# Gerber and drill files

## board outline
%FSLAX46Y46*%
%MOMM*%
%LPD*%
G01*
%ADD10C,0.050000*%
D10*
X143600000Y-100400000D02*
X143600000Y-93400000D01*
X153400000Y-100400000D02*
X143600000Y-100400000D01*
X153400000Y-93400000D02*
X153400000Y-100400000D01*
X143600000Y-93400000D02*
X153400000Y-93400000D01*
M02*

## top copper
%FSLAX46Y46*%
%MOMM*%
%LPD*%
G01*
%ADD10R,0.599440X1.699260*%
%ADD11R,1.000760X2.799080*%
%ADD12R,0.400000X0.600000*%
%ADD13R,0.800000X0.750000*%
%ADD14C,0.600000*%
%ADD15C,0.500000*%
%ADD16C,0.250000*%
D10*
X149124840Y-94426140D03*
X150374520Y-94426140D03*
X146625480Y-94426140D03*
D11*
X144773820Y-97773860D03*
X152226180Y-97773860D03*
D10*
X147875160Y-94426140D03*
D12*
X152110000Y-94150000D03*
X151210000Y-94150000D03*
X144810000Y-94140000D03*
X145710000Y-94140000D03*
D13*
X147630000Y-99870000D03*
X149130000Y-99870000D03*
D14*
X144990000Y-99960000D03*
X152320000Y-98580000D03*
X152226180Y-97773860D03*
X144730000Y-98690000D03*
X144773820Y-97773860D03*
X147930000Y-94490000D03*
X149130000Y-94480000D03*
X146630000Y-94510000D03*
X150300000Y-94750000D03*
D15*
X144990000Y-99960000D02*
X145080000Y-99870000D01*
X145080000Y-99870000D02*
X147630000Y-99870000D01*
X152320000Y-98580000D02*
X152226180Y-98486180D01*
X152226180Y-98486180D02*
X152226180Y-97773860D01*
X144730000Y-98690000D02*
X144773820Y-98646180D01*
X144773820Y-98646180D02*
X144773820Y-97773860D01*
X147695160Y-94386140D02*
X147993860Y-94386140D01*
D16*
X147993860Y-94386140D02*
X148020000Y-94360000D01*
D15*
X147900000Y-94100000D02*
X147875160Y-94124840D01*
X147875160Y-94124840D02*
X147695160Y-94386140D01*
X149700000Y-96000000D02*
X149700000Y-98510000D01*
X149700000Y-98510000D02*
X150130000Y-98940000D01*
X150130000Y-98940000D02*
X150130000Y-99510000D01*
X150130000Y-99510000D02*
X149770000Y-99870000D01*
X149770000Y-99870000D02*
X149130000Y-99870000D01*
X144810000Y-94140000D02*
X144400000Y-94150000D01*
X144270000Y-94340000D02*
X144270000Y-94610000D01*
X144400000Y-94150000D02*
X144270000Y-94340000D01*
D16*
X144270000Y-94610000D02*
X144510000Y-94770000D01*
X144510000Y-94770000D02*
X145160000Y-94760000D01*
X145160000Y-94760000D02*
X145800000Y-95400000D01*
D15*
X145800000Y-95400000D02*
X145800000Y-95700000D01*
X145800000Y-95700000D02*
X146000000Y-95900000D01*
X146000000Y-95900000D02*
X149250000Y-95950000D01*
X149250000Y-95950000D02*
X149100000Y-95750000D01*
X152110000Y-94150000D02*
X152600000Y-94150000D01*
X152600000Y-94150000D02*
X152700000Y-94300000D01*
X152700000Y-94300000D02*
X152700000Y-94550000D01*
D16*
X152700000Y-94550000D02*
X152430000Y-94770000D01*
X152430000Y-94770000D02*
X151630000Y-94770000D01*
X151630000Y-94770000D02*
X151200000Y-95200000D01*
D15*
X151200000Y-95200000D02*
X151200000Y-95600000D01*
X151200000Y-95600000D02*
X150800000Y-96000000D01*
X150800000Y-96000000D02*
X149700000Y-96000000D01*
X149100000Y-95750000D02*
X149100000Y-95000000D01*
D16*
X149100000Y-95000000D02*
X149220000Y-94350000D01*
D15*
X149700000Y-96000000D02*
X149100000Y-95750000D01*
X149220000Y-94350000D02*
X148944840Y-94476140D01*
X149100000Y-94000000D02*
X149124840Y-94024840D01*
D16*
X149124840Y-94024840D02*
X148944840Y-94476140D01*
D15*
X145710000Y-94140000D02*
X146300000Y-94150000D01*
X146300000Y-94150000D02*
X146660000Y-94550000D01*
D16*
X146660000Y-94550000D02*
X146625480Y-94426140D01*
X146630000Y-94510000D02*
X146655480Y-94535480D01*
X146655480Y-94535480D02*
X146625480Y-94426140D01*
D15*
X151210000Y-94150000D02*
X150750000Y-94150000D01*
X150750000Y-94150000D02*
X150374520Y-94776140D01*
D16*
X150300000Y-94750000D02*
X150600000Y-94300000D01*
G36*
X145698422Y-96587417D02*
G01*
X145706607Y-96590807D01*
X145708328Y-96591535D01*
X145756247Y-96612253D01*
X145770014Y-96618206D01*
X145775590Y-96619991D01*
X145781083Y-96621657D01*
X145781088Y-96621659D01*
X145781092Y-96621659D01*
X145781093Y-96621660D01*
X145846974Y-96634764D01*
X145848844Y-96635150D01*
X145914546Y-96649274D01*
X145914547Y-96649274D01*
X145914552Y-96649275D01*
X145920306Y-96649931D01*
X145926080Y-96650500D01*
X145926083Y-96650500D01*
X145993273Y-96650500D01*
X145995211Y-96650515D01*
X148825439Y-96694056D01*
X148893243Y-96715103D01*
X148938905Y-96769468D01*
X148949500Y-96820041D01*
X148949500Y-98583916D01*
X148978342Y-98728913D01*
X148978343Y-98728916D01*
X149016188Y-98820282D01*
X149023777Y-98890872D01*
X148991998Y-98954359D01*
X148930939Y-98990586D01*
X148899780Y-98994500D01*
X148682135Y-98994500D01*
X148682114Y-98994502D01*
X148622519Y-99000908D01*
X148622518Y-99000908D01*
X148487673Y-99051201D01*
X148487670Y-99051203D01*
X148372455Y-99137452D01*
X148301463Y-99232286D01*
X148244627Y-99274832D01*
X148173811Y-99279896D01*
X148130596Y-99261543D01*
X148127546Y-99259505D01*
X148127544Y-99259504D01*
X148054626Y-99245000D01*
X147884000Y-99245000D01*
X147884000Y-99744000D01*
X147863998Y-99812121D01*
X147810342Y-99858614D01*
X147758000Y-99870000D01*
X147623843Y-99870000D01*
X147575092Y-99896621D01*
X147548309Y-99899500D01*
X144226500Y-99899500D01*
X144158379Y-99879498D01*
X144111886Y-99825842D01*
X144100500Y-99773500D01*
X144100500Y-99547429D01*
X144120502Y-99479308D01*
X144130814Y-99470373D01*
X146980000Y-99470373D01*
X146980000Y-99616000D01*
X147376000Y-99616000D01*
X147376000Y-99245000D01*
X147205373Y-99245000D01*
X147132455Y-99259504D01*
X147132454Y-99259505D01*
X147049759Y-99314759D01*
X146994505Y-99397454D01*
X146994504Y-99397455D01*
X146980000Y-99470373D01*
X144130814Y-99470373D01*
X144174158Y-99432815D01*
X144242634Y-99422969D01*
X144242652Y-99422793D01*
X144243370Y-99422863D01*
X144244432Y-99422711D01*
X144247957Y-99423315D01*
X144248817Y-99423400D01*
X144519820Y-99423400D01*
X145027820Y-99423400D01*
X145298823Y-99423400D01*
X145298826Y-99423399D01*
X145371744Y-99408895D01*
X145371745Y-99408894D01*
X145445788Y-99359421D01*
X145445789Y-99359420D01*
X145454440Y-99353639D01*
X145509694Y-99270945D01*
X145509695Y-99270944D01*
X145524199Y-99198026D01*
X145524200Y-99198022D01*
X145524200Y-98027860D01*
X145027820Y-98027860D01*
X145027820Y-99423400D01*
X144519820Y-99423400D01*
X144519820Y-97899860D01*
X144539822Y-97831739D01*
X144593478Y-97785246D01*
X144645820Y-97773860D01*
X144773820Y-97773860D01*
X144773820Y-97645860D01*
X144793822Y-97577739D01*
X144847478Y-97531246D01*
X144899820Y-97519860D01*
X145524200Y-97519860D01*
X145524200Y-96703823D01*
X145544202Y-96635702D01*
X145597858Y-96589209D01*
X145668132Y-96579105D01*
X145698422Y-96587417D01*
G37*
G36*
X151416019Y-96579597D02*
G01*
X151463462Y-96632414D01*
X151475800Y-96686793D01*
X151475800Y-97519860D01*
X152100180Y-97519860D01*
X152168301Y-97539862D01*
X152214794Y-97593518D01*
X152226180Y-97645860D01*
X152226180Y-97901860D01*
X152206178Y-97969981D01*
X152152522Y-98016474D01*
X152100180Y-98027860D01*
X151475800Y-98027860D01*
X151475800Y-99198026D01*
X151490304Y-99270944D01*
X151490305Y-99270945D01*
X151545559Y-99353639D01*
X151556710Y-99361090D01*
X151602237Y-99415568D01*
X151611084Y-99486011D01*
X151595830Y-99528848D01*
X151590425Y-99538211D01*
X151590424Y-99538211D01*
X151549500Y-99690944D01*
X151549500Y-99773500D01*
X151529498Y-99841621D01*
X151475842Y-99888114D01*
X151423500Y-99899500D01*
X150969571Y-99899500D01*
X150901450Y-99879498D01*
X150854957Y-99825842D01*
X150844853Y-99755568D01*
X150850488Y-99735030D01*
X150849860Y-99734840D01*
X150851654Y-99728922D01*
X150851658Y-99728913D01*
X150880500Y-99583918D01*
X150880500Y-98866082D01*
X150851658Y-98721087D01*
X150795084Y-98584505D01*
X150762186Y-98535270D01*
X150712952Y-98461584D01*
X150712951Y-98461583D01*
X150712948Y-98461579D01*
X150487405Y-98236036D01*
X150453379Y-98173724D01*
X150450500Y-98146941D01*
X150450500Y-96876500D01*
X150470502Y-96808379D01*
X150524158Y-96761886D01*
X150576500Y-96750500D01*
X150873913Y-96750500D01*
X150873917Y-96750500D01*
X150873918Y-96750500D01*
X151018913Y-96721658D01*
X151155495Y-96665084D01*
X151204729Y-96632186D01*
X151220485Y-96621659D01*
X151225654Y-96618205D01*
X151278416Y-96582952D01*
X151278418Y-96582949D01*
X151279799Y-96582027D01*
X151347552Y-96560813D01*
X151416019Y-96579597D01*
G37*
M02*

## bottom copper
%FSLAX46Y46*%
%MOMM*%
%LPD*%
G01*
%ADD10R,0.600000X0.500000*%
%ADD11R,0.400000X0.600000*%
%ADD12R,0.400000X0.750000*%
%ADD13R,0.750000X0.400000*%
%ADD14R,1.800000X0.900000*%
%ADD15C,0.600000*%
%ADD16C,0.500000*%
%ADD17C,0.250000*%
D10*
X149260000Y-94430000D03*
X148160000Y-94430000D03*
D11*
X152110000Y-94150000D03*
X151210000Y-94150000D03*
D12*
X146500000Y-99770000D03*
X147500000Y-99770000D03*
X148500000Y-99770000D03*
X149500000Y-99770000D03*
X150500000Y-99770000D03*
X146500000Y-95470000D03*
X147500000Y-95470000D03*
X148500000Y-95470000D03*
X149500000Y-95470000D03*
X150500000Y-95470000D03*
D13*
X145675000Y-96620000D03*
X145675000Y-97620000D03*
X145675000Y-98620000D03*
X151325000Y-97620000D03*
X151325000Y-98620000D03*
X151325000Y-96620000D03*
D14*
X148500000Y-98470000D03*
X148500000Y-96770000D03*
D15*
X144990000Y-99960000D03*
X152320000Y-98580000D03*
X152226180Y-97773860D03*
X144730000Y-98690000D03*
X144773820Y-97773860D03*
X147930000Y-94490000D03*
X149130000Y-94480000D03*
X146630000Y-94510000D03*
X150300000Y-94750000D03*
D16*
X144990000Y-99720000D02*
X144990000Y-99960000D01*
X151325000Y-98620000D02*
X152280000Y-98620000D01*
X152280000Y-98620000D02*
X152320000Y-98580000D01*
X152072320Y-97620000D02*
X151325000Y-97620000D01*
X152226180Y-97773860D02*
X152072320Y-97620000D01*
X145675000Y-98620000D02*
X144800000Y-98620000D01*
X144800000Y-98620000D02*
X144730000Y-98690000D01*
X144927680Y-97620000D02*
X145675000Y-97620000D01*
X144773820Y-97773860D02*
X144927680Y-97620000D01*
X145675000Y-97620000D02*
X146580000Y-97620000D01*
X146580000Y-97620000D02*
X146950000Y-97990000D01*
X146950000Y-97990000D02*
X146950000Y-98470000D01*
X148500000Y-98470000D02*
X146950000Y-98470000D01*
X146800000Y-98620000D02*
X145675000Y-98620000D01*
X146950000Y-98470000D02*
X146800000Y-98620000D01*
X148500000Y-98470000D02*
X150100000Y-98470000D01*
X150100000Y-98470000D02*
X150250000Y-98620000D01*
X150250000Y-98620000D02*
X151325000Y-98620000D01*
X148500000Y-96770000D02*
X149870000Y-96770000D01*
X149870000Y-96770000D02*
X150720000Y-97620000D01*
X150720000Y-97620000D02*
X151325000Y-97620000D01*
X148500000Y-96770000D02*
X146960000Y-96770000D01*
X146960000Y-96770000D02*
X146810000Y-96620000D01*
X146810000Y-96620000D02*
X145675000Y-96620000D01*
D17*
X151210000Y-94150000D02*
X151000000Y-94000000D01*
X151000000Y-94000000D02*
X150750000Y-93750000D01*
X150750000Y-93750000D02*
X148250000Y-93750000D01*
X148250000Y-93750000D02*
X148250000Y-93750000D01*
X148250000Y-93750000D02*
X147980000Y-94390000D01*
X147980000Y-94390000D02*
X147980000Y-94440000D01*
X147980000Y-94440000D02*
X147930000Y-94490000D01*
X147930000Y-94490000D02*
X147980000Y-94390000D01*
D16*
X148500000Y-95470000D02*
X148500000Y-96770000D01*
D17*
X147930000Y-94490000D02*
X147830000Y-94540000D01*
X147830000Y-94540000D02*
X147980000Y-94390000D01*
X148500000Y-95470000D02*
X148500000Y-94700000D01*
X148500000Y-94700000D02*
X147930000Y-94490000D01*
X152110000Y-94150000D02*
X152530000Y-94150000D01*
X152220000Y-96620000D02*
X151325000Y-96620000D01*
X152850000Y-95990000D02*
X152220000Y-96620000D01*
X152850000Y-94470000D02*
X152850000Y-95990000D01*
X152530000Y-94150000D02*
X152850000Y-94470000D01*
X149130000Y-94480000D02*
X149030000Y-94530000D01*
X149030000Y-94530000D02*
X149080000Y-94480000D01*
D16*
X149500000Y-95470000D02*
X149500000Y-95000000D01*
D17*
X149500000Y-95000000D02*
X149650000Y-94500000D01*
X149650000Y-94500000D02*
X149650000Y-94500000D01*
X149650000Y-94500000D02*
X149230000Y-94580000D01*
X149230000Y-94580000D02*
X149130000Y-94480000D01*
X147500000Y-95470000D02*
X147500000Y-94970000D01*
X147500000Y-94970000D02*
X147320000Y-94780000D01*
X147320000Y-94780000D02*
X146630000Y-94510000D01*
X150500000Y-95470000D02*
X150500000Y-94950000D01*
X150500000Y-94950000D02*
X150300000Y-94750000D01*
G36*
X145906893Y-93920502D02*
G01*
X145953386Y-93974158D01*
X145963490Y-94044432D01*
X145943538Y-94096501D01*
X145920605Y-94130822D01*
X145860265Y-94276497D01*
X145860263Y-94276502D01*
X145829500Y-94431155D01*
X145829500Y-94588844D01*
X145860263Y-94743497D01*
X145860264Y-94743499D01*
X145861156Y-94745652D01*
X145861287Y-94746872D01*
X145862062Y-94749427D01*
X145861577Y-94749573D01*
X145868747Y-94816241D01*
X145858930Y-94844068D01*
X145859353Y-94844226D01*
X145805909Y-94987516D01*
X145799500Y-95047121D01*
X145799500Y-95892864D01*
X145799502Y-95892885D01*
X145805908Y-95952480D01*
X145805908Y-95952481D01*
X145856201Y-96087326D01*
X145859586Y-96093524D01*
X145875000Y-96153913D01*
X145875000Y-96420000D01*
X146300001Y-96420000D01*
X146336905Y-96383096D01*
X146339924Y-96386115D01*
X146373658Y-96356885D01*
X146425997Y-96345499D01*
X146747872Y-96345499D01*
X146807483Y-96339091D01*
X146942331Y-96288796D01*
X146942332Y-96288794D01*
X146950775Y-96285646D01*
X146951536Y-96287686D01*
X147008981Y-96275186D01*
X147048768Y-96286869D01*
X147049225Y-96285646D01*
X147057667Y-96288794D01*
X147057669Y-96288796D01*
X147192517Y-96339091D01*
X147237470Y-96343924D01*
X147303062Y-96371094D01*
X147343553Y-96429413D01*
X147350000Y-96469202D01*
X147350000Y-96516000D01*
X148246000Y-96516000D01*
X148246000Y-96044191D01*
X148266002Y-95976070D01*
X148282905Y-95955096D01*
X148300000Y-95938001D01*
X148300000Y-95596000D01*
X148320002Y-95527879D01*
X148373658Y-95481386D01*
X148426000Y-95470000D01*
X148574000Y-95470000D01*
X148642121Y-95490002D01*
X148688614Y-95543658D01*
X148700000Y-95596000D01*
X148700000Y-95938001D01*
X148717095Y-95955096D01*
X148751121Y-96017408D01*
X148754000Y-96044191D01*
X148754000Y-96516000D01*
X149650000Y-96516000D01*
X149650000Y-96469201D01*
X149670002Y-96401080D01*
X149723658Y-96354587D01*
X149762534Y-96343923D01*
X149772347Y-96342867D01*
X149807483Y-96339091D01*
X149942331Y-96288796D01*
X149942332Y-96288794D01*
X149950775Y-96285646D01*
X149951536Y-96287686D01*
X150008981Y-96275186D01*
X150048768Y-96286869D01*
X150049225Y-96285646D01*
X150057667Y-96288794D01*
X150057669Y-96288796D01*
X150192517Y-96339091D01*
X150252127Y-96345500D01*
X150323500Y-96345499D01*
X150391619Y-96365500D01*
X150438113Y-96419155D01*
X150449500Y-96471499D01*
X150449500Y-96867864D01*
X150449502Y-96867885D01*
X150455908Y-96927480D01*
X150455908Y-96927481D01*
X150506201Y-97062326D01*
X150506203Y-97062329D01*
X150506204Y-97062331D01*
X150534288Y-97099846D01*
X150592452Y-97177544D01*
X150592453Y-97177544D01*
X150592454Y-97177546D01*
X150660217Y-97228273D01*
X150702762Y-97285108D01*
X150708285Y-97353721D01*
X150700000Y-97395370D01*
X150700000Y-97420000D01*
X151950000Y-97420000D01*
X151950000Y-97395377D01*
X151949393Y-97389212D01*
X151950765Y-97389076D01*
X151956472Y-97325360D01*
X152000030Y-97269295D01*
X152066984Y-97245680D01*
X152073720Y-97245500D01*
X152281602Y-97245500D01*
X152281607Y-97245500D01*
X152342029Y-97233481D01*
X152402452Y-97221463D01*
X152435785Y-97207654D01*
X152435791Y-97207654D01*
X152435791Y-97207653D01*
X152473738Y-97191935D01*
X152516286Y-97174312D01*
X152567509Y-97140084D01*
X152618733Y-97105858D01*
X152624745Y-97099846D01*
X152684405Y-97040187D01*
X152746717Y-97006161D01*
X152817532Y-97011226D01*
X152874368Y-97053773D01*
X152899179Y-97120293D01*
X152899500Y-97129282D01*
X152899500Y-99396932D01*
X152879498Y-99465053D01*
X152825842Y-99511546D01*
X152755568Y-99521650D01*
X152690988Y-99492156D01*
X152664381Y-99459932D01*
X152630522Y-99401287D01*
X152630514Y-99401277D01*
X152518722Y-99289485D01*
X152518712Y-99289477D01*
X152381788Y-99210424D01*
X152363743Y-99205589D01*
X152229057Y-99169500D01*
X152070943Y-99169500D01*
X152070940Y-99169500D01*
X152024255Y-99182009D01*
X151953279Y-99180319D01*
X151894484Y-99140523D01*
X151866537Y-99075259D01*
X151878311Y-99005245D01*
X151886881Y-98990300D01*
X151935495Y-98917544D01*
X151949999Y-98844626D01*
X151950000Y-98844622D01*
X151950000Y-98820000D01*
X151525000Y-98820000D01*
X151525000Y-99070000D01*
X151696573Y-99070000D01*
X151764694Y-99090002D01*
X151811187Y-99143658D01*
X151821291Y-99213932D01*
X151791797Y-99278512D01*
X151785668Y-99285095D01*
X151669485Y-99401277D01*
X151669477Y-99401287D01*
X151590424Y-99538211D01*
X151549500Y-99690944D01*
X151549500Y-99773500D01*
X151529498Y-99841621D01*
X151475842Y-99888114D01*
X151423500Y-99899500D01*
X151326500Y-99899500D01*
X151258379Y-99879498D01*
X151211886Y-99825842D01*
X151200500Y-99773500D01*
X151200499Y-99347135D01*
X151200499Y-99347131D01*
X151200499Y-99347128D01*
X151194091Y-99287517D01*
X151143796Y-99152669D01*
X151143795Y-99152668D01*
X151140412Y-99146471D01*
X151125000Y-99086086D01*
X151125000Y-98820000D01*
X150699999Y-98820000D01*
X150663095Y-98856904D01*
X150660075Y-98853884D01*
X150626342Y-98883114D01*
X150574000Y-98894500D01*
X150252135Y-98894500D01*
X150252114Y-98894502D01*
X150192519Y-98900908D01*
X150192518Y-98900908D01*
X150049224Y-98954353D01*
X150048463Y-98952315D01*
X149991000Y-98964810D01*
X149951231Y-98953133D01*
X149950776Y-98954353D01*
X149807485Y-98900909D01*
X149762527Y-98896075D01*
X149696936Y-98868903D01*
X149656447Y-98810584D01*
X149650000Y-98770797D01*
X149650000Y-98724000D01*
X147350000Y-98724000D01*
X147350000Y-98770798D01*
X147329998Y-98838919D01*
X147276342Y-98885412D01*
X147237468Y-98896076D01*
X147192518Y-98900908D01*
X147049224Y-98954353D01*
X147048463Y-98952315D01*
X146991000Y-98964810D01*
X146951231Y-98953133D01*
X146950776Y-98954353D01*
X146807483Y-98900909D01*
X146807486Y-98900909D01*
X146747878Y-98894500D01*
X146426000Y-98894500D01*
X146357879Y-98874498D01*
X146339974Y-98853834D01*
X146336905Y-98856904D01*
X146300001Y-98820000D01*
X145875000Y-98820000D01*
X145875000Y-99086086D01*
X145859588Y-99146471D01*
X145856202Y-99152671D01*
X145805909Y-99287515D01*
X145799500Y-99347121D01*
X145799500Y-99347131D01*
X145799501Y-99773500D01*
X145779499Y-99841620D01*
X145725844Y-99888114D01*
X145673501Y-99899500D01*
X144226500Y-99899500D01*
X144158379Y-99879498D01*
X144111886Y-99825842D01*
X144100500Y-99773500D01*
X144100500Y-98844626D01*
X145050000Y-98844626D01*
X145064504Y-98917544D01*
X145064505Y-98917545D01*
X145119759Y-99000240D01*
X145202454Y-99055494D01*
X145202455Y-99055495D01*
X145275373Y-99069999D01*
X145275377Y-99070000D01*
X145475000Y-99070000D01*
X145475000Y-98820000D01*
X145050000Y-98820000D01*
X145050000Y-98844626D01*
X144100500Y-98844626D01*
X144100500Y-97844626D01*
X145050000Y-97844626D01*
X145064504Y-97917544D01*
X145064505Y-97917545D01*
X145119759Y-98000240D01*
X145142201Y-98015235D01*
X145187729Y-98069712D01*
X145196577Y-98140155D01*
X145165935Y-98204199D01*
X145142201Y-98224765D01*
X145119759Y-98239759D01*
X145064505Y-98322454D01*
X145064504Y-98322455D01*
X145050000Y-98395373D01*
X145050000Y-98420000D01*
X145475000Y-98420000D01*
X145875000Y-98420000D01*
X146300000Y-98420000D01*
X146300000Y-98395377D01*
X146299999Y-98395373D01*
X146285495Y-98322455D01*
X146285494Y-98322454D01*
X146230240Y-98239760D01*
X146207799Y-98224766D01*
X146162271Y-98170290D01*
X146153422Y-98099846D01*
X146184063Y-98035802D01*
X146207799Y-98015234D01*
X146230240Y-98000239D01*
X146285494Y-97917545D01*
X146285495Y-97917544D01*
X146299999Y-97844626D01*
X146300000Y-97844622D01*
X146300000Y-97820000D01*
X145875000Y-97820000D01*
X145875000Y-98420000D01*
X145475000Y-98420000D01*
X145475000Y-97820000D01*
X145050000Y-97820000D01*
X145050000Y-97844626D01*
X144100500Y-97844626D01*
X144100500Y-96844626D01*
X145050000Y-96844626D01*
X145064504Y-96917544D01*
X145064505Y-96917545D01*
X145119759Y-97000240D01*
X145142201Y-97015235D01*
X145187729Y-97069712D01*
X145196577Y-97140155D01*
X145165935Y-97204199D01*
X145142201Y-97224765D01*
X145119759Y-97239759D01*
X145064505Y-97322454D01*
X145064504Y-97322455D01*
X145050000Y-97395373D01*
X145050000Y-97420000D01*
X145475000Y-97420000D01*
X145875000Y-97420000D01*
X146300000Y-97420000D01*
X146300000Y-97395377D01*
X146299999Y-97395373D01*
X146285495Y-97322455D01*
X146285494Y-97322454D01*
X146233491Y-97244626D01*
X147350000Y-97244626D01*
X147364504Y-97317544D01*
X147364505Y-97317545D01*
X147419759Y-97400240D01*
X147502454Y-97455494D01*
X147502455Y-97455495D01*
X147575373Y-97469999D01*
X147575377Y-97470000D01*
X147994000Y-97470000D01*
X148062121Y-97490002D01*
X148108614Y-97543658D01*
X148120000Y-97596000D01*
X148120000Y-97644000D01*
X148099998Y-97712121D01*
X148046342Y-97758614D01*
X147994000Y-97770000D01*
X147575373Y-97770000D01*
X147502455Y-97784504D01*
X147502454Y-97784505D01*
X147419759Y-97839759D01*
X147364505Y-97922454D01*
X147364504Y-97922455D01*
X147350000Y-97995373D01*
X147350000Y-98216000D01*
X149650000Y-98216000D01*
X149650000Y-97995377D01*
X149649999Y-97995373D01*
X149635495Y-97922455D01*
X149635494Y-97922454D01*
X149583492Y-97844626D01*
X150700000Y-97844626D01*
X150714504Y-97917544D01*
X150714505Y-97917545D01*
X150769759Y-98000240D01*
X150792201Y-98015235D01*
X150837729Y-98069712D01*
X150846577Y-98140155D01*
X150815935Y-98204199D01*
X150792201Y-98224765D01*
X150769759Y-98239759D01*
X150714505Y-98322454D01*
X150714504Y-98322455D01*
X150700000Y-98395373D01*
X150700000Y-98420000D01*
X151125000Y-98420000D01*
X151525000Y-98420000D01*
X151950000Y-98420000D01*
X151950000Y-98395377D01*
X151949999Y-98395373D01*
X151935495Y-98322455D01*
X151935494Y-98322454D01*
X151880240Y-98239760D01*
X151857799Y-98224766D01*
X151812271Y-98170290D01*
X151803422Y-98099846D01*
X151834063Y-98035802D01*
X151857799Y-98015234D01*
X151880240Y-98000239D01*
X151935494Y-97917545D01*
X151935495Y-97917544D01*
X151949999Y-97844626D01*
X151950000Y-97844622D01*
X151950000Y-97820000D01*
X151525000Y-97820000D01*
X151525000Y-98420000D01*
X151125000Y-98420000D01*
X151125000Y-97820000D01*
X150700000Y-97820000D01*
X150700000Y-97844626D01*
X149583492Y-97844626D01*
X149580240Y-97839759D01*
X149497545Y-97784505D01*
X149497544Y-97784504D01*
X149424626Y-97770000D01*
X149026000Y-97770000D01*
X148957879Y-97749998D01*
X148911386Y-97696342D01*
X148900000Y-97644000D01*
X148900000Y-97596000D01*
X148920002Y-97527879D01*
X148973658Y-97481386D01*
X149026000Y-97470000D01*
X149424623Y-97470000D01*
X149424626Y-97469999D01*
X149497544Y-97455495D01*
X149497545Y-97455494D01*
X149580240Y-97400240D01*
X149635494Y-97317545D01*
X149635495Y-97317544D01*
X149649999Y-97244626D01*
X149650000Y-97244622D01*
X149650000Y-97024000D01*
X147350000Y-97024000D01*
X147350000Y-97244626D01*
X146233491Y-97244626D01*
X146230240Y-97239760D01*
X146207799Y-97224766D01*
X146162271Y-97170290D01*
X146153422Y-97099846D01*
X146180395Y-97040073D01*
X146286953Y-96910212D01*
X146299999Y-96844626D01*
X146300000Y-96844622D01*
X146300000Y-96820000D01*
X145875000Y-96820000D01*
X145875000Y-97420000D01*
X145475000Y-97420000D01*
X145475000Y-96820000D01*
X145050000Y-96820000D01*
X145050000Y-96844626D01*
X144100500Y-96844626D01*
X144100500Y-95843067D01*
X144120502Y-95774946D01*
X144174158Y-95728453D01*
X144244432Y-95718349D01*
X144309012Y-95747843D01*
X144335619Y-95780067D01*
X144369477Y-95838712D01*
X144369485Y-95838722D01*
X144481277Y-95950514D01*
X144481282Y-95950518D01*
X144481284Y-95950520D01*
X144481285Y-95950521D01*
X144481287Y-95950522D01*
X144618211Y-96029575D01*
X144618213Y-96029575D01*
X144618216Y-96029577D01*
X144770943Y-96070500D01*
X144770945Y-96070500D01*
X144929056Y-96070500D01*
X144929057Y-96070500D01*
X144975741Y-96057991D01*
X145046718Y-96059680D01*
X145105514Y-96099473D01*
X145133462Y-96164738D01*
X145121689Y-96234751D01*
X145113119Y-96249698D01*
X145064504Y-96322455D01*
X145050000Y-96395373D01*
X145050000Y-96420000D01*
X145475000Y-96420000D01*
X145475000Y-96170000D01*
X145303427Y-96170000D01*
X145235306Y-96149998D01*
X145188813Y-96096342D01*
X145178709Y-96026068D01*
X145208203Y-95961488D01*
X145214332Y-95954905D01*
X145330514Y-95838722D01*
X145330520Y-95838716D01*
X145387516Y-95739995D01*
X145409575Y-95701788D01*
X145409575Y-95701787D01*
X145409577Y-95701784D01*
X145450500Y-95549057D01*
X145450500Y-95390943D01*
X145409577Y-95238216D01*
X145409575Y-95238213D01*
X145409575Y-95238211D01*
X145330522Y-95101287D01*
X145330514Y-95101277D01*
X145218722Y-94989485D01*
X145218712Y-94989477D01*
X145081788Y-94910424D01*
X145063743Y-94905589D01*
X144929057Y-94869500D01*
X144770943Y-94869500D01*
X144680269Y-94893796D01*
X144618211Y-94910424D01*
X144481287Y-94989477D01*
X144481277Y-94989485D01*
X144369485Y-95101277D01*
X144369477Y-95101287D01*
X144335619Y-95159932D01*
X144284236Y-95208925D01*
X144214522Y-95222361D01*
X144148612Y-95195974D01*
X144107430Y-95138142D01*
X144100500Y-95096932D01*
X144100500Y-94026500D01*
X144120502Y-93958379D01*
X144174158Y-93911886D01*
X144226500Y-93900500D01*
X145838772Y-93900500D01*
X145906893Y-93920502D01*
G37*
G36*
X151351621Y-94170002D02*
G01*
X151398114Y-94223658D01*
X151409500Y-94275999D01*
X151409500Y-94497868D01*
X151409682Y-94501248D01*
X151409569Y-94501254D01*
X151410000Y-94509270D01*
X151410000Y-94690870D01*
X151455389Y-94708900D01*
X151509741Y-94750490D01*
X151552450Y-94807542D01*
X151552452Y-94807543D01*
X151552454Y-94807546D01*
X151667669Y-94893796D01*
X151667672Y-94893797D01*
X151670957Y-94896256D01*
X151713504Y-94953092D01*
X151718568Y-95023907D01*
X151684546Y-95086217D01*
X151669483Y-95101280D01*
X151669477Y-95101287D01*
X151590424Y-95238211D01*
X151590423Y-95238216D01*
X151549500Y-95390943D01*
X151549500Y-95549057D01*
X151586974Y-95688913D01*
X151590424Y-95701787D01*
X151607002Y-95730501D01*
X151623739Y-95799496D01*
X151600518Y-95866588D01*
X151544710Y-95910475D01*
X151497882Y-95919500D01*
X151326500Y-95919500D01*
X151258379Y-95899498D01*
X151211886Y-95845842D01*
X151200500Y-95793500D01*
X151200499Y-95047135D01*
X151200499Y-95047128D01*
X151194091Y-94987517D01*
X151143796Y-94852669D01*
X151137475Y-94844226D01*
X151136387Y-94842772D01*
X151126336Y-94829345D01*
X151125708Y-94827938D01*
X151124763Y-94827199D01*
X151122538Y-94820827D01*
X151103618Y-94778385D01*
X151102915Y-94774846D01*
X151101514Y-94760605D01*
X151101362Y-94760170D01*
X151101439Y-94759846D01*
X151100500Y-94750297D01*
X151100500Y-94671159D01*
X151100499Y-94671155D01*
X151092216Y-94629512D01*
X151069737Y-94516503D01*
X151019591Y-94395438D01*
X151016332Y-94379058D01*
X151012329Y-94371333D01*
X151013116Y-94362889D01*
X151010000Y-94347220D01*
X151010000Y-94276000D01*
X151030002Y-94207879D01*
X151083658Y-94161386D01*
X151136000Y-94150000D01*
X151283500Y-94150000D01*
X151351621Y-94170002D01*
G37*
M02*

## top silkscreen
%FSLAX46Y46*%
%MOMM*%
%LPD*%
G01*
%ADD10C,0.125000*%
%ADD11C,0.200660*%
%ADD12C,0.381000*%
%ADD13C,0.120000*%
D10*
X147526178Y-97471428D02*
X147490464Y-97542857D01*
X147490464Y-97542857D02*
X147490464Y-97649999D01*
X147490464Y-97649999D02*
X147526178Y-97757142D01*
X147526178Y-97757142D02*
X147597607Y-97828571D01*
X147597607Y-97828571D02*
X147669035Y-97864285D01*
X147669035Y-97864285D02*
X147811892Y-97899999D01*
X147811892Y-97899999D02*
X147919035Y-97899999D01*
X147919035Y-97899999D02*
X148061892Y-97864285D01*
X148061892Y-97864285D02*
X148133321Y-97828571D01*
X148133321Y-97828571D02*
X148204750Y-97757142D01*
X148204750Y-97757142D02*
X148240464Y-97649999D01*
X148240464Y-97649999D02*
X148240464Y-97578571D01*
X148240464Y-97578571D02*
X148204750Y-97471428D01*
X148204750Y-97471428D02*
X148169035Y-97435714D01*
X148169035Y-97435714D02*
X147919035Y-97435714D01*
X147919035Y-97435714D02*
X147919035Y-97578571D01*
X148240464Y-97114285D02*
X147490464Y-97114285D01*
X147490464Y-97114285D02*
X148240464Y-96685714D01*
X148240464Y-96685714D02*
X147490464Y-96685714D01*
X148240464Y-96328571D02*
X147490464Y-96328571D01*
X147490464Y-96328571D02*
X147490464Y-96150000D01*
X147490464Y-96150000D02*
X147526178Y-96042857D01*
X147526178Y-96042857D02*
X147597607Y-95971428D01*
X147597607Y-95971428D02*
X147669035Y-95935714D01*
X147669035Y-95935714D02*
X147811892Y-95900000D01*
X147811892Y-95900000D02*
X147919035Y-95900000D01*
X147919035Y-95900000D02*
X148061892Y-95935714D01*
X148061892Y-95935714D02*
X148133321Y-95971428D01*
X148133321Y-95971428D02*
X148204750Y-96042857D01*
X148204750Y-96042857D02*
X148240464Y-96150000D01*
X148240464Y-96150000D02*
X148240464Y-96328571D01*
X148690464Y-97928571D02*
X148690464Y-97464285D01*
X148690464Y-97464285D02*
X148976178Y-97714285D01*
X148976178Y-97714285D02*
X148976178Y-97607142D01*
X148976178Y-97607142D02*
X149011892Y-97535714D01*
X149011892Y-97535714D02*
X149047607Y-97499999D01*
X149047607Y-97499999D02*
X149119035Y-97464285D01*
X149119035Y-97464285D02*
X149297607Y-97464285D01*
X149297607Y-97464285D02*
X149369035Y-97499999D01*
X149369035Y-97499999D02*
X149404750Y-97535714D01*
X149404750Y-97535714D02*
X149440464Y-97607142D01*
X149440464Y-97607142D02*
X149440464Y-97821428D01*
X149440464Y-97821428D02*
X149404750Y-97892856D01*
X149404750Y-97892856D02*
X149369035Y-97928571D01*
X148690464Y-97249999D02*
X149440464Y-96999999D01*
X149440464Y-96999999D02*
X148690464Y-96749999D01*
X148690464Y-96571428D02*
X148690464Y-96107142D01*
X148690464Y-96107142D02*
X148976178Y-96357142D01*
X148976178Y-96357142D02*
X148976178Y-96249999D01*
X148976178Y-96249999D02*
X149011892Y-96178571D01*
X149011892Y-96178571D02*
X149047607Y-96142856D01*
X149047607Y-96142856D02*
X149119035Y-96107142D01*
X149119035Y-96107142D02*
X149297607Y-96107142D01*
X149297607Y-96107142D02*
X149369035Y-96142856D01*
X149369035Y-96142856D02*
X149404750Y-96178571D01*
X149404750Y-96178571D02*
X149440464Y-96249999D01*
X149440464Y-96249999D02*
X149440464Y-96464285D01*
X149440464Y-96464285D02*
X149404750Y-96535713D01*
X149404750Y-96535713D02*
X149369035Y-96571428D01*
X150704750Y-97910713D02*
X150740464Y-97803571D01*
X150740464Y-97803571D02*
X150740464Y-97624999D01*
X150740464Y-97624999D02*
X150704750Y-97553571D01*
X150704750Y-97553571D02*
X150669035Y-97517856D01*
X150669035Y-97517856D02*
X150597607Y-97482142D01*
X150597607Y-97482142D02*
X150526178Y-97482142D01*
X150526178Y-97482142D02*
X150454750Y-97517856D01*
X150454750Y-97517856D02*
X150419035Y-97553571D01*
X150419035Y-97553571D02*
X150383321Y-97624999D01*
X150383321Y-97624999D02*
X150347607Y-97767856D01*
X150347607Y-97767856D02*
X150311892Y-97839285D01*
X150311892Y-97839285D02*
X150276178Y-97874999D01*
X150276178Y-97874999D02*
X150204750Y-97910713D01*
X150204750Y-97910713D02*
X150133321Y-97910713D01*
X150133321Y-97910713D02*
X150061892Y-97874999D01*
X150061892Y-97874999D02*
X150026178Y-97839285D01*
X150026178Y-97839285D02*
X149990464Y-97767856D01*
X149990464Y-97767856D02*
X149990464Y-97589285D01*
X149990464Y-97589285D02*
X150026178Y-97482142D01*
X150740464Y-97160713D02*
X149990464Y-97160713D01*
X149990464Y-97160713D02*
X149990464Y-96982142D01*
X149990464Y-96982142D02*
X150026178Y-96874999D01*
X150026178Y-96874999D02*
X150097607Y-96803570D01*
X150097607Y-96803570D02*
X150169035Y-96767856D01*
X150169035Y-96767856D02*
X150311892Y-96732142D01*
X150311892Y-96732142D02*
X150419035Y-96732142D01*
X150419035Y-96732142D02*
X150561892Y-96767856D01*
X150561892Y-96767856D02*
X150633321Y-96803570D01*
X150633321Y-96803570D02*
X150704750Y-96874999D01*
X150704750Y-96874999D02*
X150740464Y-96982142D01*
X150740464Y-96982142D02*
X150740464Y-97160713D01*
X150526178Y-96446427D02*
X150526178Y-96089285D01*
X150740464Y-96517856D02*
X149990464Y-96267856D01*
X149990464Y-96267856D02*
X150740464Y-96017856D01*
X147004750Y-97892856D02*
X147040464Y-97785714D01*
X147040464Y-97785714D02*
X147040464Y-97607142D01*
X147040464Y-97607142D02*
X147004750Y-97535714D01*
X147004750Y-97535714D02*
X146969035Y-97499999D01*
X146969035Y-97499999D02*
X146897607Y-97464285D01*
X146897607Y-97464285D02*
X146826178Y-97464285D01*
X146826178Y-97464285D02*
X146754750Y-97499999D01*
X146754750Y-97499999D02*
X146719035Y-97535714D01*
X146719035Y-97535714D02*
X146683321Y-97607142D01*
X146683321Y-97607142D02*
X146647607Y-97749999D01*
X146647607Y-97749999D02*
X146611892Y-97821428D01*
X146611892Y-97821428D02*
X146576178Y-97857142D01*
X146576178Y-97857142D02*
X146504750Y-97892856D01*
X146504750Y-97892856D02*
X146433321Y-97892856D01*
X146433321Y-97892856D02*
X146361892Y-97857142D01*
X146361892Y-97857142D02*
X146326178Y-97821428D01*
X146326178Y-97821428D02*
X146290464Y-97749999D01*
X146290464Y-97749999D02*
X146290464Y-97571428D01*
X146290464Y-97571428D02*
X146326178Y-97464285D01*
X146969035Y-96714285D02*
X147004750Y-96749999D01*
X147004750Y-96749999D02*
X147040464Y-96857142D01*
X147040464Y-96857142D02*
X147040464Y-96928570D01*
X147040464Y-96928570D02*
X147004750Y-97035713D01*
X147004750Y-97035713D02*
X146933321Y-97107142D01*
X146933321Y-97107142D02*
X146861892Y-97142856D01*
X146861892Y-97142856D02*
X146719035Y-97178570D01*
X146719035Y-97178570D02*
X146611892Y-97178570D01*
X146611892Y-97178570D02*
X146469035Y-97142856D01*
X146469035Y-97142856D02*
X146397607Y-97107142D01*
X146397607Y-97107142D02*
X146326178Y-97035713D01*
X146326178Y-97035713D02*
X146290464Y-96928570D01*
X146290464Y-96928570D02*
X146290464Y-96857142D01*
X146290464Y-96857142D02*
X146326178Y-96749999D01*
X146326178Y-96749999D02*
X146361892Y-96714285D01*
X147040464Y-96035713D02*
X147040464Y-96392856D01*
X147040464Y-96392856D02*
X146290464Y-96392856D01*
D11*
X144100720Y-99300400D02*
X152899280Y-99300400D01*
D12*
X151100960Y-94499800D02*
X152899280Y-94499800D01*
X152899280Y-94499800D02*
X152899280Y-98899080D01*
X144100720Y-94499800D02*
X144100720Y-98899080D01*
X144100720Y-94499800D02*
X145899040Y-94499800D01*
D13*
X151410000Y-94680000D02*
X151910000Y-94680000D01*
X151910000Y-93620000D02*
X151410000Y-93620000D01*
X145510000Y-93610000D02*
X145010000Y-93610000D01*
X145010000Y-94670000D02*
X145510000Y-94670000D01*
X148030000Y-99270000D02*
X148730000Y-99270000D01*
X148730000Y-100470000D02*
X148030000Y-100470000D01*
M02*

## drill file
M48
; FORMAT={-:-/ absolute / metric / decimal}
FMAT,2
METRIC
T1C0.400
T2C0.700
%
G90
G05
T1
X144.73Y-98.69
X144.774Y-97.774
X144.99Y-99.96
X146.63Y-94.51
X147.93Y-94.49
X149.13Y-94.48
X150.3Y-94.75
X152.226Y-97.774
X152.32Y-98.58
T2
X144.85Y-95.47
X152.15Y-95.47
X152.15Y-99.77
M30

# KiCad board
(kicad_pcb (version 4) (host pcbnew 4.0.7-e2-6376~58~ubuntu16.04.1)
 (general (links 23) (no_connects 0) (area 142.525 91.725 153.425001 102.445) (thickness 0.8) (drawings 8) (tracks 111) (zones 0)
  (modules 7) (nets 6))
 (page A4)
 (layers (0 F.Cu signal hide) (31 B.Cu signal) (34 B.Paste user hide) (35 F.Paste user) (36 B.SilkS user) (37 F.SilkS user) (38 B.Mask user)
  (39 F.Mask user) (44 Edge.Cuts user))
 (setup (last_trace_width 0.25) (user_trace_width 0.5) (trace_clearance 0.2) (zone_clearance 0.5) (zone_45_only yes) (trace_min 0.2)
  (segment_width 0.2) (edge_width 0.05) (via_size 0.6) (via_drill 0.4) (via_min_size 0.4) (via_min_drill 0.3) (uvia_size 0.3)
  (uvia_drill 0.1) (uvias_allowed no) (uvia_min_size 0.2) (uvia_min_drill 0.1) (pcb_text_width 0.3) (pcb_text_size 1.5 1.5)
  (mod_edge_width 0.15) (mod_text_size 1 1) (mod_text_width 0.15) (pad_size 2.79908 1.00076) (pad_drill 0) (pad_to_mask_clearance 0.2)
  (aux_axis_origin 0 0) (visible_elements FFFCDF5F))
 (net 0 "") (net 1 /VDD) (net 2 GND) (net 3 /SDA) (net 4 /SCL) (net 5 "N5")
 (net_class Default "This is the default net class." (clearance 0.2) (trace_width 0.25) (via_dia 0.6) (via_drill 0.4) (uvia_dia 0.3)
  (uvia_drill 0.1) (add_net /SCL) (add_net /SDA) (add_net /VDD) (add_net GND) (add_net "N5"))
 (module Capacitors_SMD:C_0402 (layer B.Cu) (at 148.71 94.43 180)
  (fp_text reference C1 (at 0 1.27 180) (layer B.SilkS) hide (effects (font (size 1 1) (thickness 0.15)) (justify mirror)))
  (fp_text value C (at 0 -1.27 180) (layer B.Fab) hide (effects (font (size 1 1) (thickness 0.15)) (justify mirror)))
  (pad 1 smd rect (at -0.55 0 180) (size 0.6 0.5) (layers B.Cu B.Paste B.Mask) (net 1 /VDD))
  (pad 2 smd rect (at 0.55 0 180) (size 0.6 0.5) (layers B.Cu B.Paste B.Mask) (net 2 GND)))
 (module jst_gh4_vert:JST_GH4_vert (layer F.Cu) (at 148.5 96.1 90)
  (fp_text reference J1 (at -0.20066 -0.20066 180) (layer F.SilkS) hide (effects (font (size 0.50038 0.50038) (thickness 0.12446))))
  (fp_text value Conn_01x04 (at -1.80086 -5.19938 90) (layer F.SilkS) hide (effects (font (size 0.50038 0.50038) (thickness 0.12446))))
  (fp_line (start -3.2004 -4.39928) (end -3.2004 4.39928) (layer F.SilkS) (width 0.20066))
  (fp_line (start 1.6002 2.60096) (end 1.6002 4.39928) (layer F.SilkS) (width 0.381))
  (fp_line (start 1.6002 4.39928) (end -2.79908 4.39928) (layer F.SilkS) (width 0.381))
  (fp_line (start 1.6002 -4.39928) (end -2.79908 -4.39928) (layer F.SilkS) (width 0.381))
  (fp_line (start 1.6002 -4.39928) (end 1.6002 -2.60096) (layer F.SilkS) (width 0.381))
  (pad 3 smd rect (at 1.67386 0.62484) (size 0.59944 1.69926) (layers F.Cu F.Paste F.Mask) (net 1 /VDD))
  (pad 4 smd rect (at 1.67386 1.87452) (size 0.59944 1.69926) (layers F.Cu F.Paste F.Mask) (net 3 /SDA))
  (pad 1 smd rect (at 1.67386 -1.87452) (size 0.59944 1.69926) (layers F.Cu F.Paste F.Mask) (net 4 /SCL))
  (pad "" smd rect (at -1.67386 -3.72618 90) (size 2.79908 1.00076) (layers F.Cu F.Paste F.Mask) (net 2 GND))
  (pad "" smd rect (at -1.67386 3.72618 90) (size 2.79908 1.00076) (layers F.Cu F.Paste F.Mask) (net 2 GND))
  (pad 2 smd rect (at 1.67386 -0.62484) (size 0.59944 1.69926) (layers F.Cu F.Paste F.Mask) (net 2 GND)))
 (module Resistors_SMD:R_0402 (layer F.Cu) (at 151.66 94.15 180)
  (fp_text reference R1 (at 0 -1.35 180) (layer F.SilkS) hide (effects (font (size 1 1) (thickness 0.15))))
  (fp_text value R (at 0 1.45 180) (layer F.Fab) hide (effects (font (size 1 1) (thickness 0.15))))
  (fp_line (start 0.25 -0.53) (end -0.25 -0.53) (layer F.SilkS) (width 0.12))
  (fp_line (start -0.25 0.53) (end 0.25 0.53) (layer F.SilkS) (width 0.12))
  (pad 1 smd rect (at -0.45 0 180) (size 0.4 0.6) (layers F.Cu F.Paste F.Mask) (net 1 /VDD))
  (pad 2 smd rect (at 0.45 0 180) (size 0.4 0.6) (layers F.Cu F.Paste F.Mask) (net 3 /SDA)))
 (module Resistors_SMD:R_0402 (layer F.Cu) (at 145.26 94.14)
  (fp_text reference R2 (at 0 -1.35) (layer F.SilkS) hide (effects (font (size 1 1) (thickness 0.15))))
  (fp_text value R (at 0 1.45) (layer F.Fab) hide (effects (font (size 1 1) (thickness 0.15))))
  (fp_line (start 0.25 -0.53) (end -0.25 -0.53) (layer F.SilkS) (width 0.12))
  (fp_line (start -0.25 0.53) (end 0.25 0.53) (layer F.SilkS) (width 0.12))
  (pad 1 smd rect (at -0.45 0) (size 0.4 0.6) (layers F.Cu F.Paste F.Mask) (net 1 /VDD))
  (pad 2 smd rect (at 0.45 0) (size 0.4 0.6) (layers F.Cu F.Paste F.Mask) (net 4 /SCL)))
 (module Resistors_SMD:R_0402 (layer B.Cu) (at 151.66 94.15 180)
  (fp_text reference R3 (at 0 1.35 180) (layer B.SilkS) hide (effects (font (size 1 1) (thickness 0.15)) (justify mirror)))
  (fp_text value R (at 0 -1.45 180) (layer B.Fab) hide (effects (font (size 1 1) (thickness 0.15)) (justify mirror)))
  (pad 1 smd rect (at -0.45 0 180) (size 0.4 0.6) (layers B.Cu B.Paste B.Mask) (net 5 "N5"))
  (pad 2 smd rect (at 0.45 0 180) (size 0.4 0.6) (layers B.Cu B.Paste B.Mask) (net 2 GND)))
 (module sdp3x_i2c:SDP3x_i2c (layer B.Cu) (at 148.5 97.62)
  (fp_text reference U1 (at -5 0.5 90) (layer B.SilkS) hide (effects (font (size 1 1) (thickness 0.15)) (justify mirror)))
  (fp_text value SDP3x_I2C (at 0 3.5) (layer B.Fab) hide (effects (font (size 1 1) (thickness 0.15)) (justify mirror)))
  (pad 16 smd rect (at -2 2.15) (size 0.4 0.75) (layers B.Cu B.Paste B.Mask))
  (pad 15 smd rect (at -1 2.15) (size 0.4 0.75) (layers B.Cu B.Paste B.Mask))
  (pad 14 smd rect (at 0 2.15) (size 0.4 0.75) (layers B.Cu B.Paste B.Mask))
  (pad 13 smd rect (at 1 2.15) (size 0.4 0.75) (layers B.Cu B.Paste B.Mask))
  (pad 12 smd rect (at 2 2.15) (size 0.4 0.75) (layers B.Cu B.Paste B.Mask))
  (pad 4 smd rect (at -2 -2.15) (size 0.4 0.75) (layers B.Cu B.Paste B.Mask))
  (pad 5 smd rect (at -1 -2.15) (size 0.4 0.75) (layers B.Cu B.Paste B.Mask) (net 4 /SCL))
  (pad 6 smd rect (at 0 -2.15) (size 0.4 0.75) (layers B.Cu B.Paste B.Mask) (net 2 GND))
  (pad 7 smd rect (at 1 -2.15) (size 0.4 0.75) (layers B.Cu B.Paste B.Mask) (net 1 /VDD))
  (pad 8 smd rect (at 2 -2.15) (size 0.4 0.75) (layers B.Cu B.Paste B.Mask) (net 3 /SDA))
  (pad 3 smd rect (at -2.825 -1) (size 0.75 0.4) (layers B.Cu B.Paste B.Mask) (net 2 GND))
  (pad 2 smd rect (at -2.825 0) (size 0.75 0.4) (layers B.Cu B.Paste B.Mask) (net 2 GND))
  (pad 1 smd rect (at -2.825 1) (size 0.75 0.4) (layers B.Cu B.Paste B.Mask) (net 2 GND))
  (pad 10 smd rect (at 2.825 0) (size 0.75 0.4) (layers B.Cu B.Paste B.Mask) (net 2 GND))
  (pad 11 smd rect (at 2.825 1) (size 0.75 0.4) (layers B.Cu B.Paste B.Mask) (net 2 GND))
  (pad 9 smd rect (at 2.825 -1) (size 0.75 0.4) (layers B.Cu B.Paste B.Mask) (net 5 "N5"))
  (pad 1 smd rect (at 0 0.85) (size 1.8 0.9) (layers B.Cu B.Paste B.Mask) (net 2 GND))
  (pad 1 smd rect (at 0 -0.85) (size 1.8 0.9) (layers B.Cu B.Paste B.Mask) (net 2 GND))
  (pad "" np_thru_hole circle (at 3.65 -2.15) (size 0.7 0.7) (drill 0.7) (layers *.Cu *.Mask) (zone_connect 0))
  (pad "" np_thru_hole circle (at 3.65 2.15) (size 0.7 0.7) (drill 0.7) (layers *.Cu *.Mask))
  (pad "" np_thru_hole circle (at -3.65 -2.15) (size 0.7 0.7) (drill 0.7) (layers *.Cu *.Mask)))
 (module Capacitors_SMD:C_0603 (layer F.Cu) (at 148.38 99.87 180)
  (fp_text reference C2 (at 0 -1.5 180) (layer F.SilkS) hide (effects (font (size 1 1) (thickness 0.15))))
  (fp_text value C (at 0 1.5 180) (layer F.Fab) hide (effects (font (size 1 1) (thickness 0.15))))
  (fp_line (start 0.35 0.6) (end -0.35 0.6) (layer F.SilkS) (width 0.12))
  (fp_line (start -0.35 -0.6) (end 0.35 -0.6) (layer F.SilkS) (width 0.12))
  (pad 2 smd rect (at 0.75 0 180) (size 0.8 0.75) (layers F.Cu F.Paste F.Mask) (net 2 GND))
  (pad 1 smd rect (at -0.75 0 180) (size 0.8 0.75) (layers F.Cu F.Paste F.Mask) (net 1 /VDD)))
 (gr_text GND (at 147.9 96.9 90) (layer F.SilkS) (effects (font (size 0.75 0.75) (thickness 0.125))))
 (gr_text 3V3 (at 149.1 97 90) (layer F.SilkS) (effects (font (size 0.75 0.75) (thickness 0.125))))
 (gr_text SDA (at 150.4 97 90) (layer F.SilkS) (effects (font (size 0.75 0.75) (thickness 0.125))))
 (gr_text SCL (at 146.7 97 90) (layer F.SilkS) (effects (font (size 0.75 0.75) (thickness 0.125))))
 (gr_line (start 143.6 100.4) (end 143.6 93.4) (angle 90) (layer Edge.Cuts) (width 0.05))
 (gr_line (start 153.4 100.4) (end 143.6 100.4) (angle 90) (layer Edge.Cuts) (width 0.05))
 (gr_line (start 153.4 93.4) (end 153.4 100.4) (angle 90) (layer Edge.Cuts) (width 0.05))
 (gr_line (start 143.6 93.4) (end 153.4 93.4) (angle 90) (layer Edge.Cuts) (width 0.05))
 (segment (start 144.99 99.72) (end 144.99 99.96) (width 0.5) (layer B.Cu) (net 2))
 (via (at 144.99 99.96) (size 0.6) (drill 0.4) (layers F.Cu B.Cu) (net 2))
 (segment (start 144.99 99.96) (end 145.08 99.87) (width 0.5) (layer F.Cu) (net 2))
 (segment (start 145.08 99.87) (end 147.63 99.87) (width 0.5) (layer F.Cu) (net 2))
 (segment (start 151.325 98.62) (end 152.28 98.62) (width 0.5) (layer B.Cu) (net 2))
 (segment (start 152.28 98.62) (end 152.32 98.58) (width 0.5) (layer B.Cu) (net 2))
 (via (at 152.32 98.58) (size 0.6) (drill 0.4) (layers F.Cu B.Cu) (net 2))
 (segment (start 152.32 98.58) (end 152.22618 98.48618) (width 0.5) (layer F.Cu) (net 2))
 (segment (start 152.22618 98.48618) (end 152.22618 97.77386) (width 0.5) (layer F.Cu) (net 2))
 (segment (start 152.07232 97.62) (end 151.325 97.62) (width 0.5) (layer B.Cu) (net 2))
 (segment (start 152.22618 97.77386) (end 152.07232 97.62) (width 0.5) (layer B.Cu) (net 2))
 (via (at 152.22618 97.77386) (size 0.6) (drill 0.4) (layers F.Cu B.Cu) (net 2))
 (segment (start 145.675 98.62) (end 144.8 98.62) (width 0.5) (layer B.Cu) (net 2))
 (segment (start 144.8 98.62) (end 144.73 98.69) (width 0.5) (layer B.Cu) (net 2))
 (via (at 144.73 98.69) (size 0.6) (drill 0.4) (layers F.Cu B.Cu) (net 2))
 (segment (start 144.73 98.69) (end 144.77382 98.64618) (width 0.5) (layer F.Cu) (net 2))
 (segment (start 144.77382 98.64618) (end 144.77382 97.77386) (width 0.5) (layer F.Cu) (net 2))
 (segment (start 144.92768 97.62) (end 145.675 97.62) (width 0.5) (layer B.Cu) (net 2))
 (segment (start 144.77382 97.77386) (end 144.92768 97.62) (width 0.5) (layer B.Cu) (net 2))
 (via (at 144.77382 97.77386) (size 0.6) (drill 0.4) (layers F.Cu B.Cu) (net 2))
 (segment (start 145.675 97.62) (end 146.58 97.62) (width 0.5) (layer B.Cu) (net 2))
 (segment (start 146.58 97.62) (end 146.95 97.99) (width 0.5) (layer B.Cu) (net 2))
 (segment (start 146.95 97.99) (end 146.95 98.47) (width 0.5) (layer B.Cu) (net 2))
 (segment (start 148.5 98.47) (end 146.95 98.47) (width 0.5) (layer B.Cu) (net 2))
 (segment (start 146.8 98.62) (end 145.675 98.62) (width 0.5) (layer B.Cu) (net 2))
 (segment (start 146.95 98.47) (end 146.8 98.62) (width 0.5) (layer B.Cu) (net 2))
 (segment (start 148.5 98.47) (end 150.1 98.47) (width 0.5) (layer B.Cu) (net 2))
 (segment (start 150.1 98.47) (end 150.25 98.62) (width 0.5) (layer B.Cu) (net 2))
 (segment (start 150.25 98.62) (end 151.325 98.62) (width 0.5) (layer B.Cu) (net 2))
 (segment (start 148.5 96.77) (end 149.87 96.77) (width 0.5) (layer B.Cu) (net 2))
 (segment (start 149.87 96.77) (end 150.72 97.62) (width 0.5) (layer B.Cu) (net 2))
 (segment (start 150.72 97.62) (end 151.325 97.62) (width 0.5) (layer B.Cu) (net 2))
 (segment (start 148.5 96.77) (end 146.96 96.77) (width 0.5) (layer B.Cu) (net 2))
 (segment (start 146.96 96.77) (end 146.81 96.62) (width 0.5) (layer B.Cu) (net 2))
 (segment (start 146.81 96.62) (end 145.675 96.62) (width 0.5) (layer B.Cu) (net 2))
 (segment (start 151.21 94.15) (end 151 94) (width 0.25) (layer B.Cu) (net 2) (status 10))
 (segment (start 151 94) (end 150.75 93.75) (width 0.25) (layer B.Cu) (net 2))
 (segment (start 150.75 93.75) (end 148.25 93.75) (width 0.25) (layer B.Cu) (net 2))
 (segment (start 148.25 93.75) (end 148.25 93.75) (width 0.25) (layer B.Cu) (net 2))
 (segment (start 148.25 93.75) (end 147.98 94.39) (width 0.25) (layer B.Cu) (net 2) (status 20))
 (segment (start 147.69516 94.38614) (end 147.99386 94.38614) (width 0.5) (layer F.Cu) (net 2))
 (segment (start 147.99386 94.38614) (end 148.02 94.36) (width 0.25) (layer F.Cu) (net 2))
 (via (at 147.93 94.49) (size 0.6) (drill 0.4) (layers F.Cu B.Cu) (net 2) (status 30))
 (segment (start 147.98 94.39) (end 147.98 94.44) (width 0.25) (layer B.Cu) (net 2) (status 30))
 (segment (start 147.98 94.44) (end 147.93 94.49) (width 0.25) (layer B.Cu) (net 2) (status 30))
 (segment (start 147.93 94.49) (end 147.98 94.39) (width 0.25) (layer B.Cu) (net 2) (status 30))
 (segment (start 148.5 95.47) (end 148.5 96.77) (width 0.5) (layer B.Cu) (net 2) (status 30))
 (segment (start 147.9 94.1) (end 147.87516 94.12484) (width 0.5) (layer F.Cu) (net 2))
 (segment (start 147.87516 94.12484) (end 147.69516 94.38614) (width 0.5) (layer F.Cu) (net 2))
 (segment (start 147.93 94.49) (end 147.83 94.54) (width 0.25) (layer B.Cu) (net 2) (status 30))
 (segment (start 147.83 94.54) (end 147.98 94.39) (width 0.25) (layer B.Cu) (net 2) (status 30))
 (segment (start 148.5 95.47) (end 148.5 94.7) (width 0.25) (layer B.Cu) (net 2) (status 10))
 (segment (start 148.5 94.7) (end 147.93 94.49) (width 0.25) (layer B.Cu) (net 2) (status 20))
 (segment (start 152.11 94.15) (end 152.53 94.15) (width 0.25) (layer B.Cu) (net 5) (status 10))
 (segment (start 152.22 96.62) (end 151.325 96.62) (width 0.25) (layer B.Cu) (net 5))
 (segment (start 152.85 95.99) (end 152.22 96.62) (width 0.25) (layer B.Cu) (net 5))
 (segment (start 152.85 94.47) (end 152.85 95.99) (width 0.25) (layer B.Cu) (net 5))
 (segment (start 152.53 94.15) (end 152.85 94.47) (width 0.25) (layer B.Cu) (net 5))
 (segment (start 149.7 96) (end 149.7 98.51) (width 0.5) (layer F.Cu) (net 1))
 (segment (start 149.7 98.51) (end 150.13 98.94) (width 0.5) (layer F.Cu) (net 1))
 (segment (start 150.13 98.94) (end 150.13 99.51) (width 0.5) (layer F.Cu) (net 1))
 (segment (start 150.13 99.51) (end 149.77 99.87) (width 0.5) (layer F.Cu) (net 1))
 (segment (start 149.77 99.87) (end 149.13 99.87) (width 0.5) (layer F.Cu) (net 1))
 (segment (start 144.81 94.14) (end 144.4 94.15) (width 0.5) (layer F.Cu) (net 1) (status 10))
 (segment (start 144.27 94.34) (end 144.27 94.61) (width 0.5) (layer F.Cu) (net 1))
 (segment (start 144.4 94.15) (end 144.27 94.34) (width 0.5) (layer F.Cu) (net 1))
 (segment (start 144.27 94.61) (end 144.51 94.77) (width 0.25) (layer F.Cu) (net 1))
 (segment (start 144.51 94.77) (end 145.16 94.76) (width 0.25) (layer F.Cu) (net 1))
 (segment (start 145.16 94.76) (end 145.8 95.4) (width 0.25) (layer F.Cu) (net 1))
 (segment (start 145.8 95.4) (end 145.8 95.7) (width 0.5) (layer F.Cu) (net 1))
 (segment (start 145.8 95.7) (end 146 95.9) (width 0.5) (layer F.Cu) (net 1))
 (segment (start 146 95.9) (end 149.25 95.95) (width 0.5) (layer F.Cu) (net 1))
 (segment (start 149.25 95.95) (end 149.1 95.75) (width 0.5) (layer F.Cu) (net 1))
 (segment (start 152.11 94.15) (end 152.6 94.15) (width 0.5) (layer F.Cu) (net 1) (status 10))
 (segment (start 152.6 94.15) (end 152.7 94.3) (width 0.5) (layer F.Cu) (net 1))
 (segment (start 152.7 94.3) (end 152.7 94.55) (width 0.5) (layer F.Cu) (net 1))
 (segment (start 152.7 94.55) (end 152.43 94.77) (width 0.25) (layer F.Cu) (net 1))
 (segment (start 152.43 94.77) (end 151.63 94.77) (width 0.25) (layer F.Cu) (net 1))
 (segment (start 151.63 94.77) (end 151.2 95.2) (width 0.25) (layer F.Cu) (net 1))
 (segment (start 151.2 95.2) (end 151.2 95.6) (width 0.5) (layer F.Cu) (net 1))
 (segment (start 151.2 95.6) (end 150.8 96) (width 0.5) (layer F.Cu) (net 1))
 (segment (start 150.8 96) (end 149.7 96) (width 0.5) (layer F.Cu) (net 1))
 (segment (start 149.1 95.75) (end 149.1 95) (width 0.5) (layer F.Cu) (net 1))
 (segment (start 149.1 95) (end 149.22 94.35) (width 0.25) (layer F.Cu) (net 1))
 (segment (start 149.7 96) (end 149.1 95.75) (width 0.5) (layer F.Cu) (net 1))
 (segment (start 149.22 94.35) (end 148.94484 94.47614) (width 0.5) (layer F.Cu) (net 1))
 (segment (start 149.1 94) (end 149.12484 94.02484) (width 0.5) (layer F.Cu) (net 1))
 (segment (start 149.12484 94.02484) (end 148.94484 94.47614) (width 0.25) (layer F.Cu) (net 1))
 (segment (start 149.13 94.48) (end 149.03 94.53) (width 0.25) (layer B.Cu) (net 1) (status 30))
 (segment (start 149.03 94.53) (end 149.08 94.48) (width 0.25) (layer B.Cu) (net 1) (status 30))
 (segment (start 149.5 95.47) (end 149.5 95) (width 0.5) (layer B.Cu) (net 1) (status 20))
 (segment (start 149.5 95) (end 149.65 94.5) (width 0.25) (layer B.Cu) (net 1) (status 20))
 (segment (start 149.65 94.5) (end 149.65 94.5) (width 0.25) (layer B.Cu) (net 1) (status 20))
 (segment (start 149.65 94.5) (end 149.23 94.58) (width 0.25) (layer B.Cu) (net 1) (status 20))
 (via (at 149.13 94.48) (size 0.6) (drill 0.4) (layers F.Cu B.Cu) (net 1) (status 30))
 (segment (start 149.23 94.58) (end 149.13 94.48) (width 0.25) (layer B.Cu) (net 1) (status 30))
 (segment (start 145.71 94.14) (end 146.3 94.15) (width 0.5) (layer F.Cu) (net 4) (status 10))
 (segment (start 146.3 94.15) (end 146.66 94.55) (width 0.5) (layer F.Cu) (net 4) (status 10))
 (segment (start 146.66 94.55) (end 146.62548 94.42614) (width 0.25) (layer F.Cu) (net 4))
 (segment (start 147.5 95.47) (end 147.5 94.97) (width 0.25) (layer B.Cu) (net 4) (status 30))
 (segment (start 147.5 94.97) (end 147.32 94.78) (width 0.25) (layer B.Cu) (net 4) (status 10))
 (segment (start 147.32 94.78) (end 146.63 94.51) (width 0.25) (layer B.Cu) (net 4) (status 10))
 (via (at 146.63 94.51) (size 0.6) (drill 0.4) (layers F.Cu B.Cu) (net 4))
 (segment (start 146.63 94.51) (end 146.65548 94.53548) (width 0.25) (layer F.Cu) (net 4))
 (segment (start 146.65548 94.53548) (end 146.62548 94.42614) (width 0.25) (layer F.Cu) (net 4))
 (segment (start 151.21 94.15) (end 150.75 94.15) (width 0.5) (layer F.Cu) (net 3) (status 10))
 (segment (start 150.75 94.15) (end 150.37452 94.77614) (width 0.5) (layer F.Cu) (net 3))
 (segment (start 150.5 95.47) (end 150.5 94.95) (width 0.25) (layer B.Cu) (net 3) (status 10))
 (segment (start 150.3 94.75) (end 150.6 94.3) (width 0.25) (layer F.Cu) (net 3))
 (via (at 150.3 94.75) (size 0.6) (drill 0.4) (layers F.Cu B.Cu) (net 3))
 (segment (start 150.5 94.95) (end 150.3 94.75) (width 0.25) (layer B.Cu) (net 3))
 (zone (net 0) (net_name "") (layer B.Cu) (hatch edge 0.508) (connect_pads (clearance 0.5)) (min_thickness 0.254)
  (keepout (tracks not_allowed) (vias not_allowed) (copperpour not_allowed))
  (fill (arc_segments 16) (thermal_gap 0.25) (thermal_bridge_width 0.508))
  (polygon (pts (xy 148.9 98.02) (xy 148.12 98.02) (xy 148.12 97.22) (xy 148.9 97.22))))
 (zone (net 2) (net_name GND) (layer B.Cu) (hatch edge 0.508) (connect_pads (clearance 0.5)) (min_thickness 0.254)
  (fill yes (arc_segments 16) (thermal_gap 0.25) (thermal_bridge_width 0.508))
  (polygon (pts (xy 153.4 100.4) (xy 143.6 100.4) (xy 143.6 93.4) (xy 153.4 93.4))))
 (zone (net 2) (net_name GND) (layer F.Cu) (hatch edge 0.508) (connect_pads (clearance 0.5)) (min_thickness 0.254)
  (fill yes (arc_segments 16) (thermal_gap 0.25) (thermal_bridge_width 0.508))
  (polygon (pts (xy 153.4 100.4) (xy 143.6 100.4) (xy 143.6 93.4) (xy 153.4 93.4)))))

